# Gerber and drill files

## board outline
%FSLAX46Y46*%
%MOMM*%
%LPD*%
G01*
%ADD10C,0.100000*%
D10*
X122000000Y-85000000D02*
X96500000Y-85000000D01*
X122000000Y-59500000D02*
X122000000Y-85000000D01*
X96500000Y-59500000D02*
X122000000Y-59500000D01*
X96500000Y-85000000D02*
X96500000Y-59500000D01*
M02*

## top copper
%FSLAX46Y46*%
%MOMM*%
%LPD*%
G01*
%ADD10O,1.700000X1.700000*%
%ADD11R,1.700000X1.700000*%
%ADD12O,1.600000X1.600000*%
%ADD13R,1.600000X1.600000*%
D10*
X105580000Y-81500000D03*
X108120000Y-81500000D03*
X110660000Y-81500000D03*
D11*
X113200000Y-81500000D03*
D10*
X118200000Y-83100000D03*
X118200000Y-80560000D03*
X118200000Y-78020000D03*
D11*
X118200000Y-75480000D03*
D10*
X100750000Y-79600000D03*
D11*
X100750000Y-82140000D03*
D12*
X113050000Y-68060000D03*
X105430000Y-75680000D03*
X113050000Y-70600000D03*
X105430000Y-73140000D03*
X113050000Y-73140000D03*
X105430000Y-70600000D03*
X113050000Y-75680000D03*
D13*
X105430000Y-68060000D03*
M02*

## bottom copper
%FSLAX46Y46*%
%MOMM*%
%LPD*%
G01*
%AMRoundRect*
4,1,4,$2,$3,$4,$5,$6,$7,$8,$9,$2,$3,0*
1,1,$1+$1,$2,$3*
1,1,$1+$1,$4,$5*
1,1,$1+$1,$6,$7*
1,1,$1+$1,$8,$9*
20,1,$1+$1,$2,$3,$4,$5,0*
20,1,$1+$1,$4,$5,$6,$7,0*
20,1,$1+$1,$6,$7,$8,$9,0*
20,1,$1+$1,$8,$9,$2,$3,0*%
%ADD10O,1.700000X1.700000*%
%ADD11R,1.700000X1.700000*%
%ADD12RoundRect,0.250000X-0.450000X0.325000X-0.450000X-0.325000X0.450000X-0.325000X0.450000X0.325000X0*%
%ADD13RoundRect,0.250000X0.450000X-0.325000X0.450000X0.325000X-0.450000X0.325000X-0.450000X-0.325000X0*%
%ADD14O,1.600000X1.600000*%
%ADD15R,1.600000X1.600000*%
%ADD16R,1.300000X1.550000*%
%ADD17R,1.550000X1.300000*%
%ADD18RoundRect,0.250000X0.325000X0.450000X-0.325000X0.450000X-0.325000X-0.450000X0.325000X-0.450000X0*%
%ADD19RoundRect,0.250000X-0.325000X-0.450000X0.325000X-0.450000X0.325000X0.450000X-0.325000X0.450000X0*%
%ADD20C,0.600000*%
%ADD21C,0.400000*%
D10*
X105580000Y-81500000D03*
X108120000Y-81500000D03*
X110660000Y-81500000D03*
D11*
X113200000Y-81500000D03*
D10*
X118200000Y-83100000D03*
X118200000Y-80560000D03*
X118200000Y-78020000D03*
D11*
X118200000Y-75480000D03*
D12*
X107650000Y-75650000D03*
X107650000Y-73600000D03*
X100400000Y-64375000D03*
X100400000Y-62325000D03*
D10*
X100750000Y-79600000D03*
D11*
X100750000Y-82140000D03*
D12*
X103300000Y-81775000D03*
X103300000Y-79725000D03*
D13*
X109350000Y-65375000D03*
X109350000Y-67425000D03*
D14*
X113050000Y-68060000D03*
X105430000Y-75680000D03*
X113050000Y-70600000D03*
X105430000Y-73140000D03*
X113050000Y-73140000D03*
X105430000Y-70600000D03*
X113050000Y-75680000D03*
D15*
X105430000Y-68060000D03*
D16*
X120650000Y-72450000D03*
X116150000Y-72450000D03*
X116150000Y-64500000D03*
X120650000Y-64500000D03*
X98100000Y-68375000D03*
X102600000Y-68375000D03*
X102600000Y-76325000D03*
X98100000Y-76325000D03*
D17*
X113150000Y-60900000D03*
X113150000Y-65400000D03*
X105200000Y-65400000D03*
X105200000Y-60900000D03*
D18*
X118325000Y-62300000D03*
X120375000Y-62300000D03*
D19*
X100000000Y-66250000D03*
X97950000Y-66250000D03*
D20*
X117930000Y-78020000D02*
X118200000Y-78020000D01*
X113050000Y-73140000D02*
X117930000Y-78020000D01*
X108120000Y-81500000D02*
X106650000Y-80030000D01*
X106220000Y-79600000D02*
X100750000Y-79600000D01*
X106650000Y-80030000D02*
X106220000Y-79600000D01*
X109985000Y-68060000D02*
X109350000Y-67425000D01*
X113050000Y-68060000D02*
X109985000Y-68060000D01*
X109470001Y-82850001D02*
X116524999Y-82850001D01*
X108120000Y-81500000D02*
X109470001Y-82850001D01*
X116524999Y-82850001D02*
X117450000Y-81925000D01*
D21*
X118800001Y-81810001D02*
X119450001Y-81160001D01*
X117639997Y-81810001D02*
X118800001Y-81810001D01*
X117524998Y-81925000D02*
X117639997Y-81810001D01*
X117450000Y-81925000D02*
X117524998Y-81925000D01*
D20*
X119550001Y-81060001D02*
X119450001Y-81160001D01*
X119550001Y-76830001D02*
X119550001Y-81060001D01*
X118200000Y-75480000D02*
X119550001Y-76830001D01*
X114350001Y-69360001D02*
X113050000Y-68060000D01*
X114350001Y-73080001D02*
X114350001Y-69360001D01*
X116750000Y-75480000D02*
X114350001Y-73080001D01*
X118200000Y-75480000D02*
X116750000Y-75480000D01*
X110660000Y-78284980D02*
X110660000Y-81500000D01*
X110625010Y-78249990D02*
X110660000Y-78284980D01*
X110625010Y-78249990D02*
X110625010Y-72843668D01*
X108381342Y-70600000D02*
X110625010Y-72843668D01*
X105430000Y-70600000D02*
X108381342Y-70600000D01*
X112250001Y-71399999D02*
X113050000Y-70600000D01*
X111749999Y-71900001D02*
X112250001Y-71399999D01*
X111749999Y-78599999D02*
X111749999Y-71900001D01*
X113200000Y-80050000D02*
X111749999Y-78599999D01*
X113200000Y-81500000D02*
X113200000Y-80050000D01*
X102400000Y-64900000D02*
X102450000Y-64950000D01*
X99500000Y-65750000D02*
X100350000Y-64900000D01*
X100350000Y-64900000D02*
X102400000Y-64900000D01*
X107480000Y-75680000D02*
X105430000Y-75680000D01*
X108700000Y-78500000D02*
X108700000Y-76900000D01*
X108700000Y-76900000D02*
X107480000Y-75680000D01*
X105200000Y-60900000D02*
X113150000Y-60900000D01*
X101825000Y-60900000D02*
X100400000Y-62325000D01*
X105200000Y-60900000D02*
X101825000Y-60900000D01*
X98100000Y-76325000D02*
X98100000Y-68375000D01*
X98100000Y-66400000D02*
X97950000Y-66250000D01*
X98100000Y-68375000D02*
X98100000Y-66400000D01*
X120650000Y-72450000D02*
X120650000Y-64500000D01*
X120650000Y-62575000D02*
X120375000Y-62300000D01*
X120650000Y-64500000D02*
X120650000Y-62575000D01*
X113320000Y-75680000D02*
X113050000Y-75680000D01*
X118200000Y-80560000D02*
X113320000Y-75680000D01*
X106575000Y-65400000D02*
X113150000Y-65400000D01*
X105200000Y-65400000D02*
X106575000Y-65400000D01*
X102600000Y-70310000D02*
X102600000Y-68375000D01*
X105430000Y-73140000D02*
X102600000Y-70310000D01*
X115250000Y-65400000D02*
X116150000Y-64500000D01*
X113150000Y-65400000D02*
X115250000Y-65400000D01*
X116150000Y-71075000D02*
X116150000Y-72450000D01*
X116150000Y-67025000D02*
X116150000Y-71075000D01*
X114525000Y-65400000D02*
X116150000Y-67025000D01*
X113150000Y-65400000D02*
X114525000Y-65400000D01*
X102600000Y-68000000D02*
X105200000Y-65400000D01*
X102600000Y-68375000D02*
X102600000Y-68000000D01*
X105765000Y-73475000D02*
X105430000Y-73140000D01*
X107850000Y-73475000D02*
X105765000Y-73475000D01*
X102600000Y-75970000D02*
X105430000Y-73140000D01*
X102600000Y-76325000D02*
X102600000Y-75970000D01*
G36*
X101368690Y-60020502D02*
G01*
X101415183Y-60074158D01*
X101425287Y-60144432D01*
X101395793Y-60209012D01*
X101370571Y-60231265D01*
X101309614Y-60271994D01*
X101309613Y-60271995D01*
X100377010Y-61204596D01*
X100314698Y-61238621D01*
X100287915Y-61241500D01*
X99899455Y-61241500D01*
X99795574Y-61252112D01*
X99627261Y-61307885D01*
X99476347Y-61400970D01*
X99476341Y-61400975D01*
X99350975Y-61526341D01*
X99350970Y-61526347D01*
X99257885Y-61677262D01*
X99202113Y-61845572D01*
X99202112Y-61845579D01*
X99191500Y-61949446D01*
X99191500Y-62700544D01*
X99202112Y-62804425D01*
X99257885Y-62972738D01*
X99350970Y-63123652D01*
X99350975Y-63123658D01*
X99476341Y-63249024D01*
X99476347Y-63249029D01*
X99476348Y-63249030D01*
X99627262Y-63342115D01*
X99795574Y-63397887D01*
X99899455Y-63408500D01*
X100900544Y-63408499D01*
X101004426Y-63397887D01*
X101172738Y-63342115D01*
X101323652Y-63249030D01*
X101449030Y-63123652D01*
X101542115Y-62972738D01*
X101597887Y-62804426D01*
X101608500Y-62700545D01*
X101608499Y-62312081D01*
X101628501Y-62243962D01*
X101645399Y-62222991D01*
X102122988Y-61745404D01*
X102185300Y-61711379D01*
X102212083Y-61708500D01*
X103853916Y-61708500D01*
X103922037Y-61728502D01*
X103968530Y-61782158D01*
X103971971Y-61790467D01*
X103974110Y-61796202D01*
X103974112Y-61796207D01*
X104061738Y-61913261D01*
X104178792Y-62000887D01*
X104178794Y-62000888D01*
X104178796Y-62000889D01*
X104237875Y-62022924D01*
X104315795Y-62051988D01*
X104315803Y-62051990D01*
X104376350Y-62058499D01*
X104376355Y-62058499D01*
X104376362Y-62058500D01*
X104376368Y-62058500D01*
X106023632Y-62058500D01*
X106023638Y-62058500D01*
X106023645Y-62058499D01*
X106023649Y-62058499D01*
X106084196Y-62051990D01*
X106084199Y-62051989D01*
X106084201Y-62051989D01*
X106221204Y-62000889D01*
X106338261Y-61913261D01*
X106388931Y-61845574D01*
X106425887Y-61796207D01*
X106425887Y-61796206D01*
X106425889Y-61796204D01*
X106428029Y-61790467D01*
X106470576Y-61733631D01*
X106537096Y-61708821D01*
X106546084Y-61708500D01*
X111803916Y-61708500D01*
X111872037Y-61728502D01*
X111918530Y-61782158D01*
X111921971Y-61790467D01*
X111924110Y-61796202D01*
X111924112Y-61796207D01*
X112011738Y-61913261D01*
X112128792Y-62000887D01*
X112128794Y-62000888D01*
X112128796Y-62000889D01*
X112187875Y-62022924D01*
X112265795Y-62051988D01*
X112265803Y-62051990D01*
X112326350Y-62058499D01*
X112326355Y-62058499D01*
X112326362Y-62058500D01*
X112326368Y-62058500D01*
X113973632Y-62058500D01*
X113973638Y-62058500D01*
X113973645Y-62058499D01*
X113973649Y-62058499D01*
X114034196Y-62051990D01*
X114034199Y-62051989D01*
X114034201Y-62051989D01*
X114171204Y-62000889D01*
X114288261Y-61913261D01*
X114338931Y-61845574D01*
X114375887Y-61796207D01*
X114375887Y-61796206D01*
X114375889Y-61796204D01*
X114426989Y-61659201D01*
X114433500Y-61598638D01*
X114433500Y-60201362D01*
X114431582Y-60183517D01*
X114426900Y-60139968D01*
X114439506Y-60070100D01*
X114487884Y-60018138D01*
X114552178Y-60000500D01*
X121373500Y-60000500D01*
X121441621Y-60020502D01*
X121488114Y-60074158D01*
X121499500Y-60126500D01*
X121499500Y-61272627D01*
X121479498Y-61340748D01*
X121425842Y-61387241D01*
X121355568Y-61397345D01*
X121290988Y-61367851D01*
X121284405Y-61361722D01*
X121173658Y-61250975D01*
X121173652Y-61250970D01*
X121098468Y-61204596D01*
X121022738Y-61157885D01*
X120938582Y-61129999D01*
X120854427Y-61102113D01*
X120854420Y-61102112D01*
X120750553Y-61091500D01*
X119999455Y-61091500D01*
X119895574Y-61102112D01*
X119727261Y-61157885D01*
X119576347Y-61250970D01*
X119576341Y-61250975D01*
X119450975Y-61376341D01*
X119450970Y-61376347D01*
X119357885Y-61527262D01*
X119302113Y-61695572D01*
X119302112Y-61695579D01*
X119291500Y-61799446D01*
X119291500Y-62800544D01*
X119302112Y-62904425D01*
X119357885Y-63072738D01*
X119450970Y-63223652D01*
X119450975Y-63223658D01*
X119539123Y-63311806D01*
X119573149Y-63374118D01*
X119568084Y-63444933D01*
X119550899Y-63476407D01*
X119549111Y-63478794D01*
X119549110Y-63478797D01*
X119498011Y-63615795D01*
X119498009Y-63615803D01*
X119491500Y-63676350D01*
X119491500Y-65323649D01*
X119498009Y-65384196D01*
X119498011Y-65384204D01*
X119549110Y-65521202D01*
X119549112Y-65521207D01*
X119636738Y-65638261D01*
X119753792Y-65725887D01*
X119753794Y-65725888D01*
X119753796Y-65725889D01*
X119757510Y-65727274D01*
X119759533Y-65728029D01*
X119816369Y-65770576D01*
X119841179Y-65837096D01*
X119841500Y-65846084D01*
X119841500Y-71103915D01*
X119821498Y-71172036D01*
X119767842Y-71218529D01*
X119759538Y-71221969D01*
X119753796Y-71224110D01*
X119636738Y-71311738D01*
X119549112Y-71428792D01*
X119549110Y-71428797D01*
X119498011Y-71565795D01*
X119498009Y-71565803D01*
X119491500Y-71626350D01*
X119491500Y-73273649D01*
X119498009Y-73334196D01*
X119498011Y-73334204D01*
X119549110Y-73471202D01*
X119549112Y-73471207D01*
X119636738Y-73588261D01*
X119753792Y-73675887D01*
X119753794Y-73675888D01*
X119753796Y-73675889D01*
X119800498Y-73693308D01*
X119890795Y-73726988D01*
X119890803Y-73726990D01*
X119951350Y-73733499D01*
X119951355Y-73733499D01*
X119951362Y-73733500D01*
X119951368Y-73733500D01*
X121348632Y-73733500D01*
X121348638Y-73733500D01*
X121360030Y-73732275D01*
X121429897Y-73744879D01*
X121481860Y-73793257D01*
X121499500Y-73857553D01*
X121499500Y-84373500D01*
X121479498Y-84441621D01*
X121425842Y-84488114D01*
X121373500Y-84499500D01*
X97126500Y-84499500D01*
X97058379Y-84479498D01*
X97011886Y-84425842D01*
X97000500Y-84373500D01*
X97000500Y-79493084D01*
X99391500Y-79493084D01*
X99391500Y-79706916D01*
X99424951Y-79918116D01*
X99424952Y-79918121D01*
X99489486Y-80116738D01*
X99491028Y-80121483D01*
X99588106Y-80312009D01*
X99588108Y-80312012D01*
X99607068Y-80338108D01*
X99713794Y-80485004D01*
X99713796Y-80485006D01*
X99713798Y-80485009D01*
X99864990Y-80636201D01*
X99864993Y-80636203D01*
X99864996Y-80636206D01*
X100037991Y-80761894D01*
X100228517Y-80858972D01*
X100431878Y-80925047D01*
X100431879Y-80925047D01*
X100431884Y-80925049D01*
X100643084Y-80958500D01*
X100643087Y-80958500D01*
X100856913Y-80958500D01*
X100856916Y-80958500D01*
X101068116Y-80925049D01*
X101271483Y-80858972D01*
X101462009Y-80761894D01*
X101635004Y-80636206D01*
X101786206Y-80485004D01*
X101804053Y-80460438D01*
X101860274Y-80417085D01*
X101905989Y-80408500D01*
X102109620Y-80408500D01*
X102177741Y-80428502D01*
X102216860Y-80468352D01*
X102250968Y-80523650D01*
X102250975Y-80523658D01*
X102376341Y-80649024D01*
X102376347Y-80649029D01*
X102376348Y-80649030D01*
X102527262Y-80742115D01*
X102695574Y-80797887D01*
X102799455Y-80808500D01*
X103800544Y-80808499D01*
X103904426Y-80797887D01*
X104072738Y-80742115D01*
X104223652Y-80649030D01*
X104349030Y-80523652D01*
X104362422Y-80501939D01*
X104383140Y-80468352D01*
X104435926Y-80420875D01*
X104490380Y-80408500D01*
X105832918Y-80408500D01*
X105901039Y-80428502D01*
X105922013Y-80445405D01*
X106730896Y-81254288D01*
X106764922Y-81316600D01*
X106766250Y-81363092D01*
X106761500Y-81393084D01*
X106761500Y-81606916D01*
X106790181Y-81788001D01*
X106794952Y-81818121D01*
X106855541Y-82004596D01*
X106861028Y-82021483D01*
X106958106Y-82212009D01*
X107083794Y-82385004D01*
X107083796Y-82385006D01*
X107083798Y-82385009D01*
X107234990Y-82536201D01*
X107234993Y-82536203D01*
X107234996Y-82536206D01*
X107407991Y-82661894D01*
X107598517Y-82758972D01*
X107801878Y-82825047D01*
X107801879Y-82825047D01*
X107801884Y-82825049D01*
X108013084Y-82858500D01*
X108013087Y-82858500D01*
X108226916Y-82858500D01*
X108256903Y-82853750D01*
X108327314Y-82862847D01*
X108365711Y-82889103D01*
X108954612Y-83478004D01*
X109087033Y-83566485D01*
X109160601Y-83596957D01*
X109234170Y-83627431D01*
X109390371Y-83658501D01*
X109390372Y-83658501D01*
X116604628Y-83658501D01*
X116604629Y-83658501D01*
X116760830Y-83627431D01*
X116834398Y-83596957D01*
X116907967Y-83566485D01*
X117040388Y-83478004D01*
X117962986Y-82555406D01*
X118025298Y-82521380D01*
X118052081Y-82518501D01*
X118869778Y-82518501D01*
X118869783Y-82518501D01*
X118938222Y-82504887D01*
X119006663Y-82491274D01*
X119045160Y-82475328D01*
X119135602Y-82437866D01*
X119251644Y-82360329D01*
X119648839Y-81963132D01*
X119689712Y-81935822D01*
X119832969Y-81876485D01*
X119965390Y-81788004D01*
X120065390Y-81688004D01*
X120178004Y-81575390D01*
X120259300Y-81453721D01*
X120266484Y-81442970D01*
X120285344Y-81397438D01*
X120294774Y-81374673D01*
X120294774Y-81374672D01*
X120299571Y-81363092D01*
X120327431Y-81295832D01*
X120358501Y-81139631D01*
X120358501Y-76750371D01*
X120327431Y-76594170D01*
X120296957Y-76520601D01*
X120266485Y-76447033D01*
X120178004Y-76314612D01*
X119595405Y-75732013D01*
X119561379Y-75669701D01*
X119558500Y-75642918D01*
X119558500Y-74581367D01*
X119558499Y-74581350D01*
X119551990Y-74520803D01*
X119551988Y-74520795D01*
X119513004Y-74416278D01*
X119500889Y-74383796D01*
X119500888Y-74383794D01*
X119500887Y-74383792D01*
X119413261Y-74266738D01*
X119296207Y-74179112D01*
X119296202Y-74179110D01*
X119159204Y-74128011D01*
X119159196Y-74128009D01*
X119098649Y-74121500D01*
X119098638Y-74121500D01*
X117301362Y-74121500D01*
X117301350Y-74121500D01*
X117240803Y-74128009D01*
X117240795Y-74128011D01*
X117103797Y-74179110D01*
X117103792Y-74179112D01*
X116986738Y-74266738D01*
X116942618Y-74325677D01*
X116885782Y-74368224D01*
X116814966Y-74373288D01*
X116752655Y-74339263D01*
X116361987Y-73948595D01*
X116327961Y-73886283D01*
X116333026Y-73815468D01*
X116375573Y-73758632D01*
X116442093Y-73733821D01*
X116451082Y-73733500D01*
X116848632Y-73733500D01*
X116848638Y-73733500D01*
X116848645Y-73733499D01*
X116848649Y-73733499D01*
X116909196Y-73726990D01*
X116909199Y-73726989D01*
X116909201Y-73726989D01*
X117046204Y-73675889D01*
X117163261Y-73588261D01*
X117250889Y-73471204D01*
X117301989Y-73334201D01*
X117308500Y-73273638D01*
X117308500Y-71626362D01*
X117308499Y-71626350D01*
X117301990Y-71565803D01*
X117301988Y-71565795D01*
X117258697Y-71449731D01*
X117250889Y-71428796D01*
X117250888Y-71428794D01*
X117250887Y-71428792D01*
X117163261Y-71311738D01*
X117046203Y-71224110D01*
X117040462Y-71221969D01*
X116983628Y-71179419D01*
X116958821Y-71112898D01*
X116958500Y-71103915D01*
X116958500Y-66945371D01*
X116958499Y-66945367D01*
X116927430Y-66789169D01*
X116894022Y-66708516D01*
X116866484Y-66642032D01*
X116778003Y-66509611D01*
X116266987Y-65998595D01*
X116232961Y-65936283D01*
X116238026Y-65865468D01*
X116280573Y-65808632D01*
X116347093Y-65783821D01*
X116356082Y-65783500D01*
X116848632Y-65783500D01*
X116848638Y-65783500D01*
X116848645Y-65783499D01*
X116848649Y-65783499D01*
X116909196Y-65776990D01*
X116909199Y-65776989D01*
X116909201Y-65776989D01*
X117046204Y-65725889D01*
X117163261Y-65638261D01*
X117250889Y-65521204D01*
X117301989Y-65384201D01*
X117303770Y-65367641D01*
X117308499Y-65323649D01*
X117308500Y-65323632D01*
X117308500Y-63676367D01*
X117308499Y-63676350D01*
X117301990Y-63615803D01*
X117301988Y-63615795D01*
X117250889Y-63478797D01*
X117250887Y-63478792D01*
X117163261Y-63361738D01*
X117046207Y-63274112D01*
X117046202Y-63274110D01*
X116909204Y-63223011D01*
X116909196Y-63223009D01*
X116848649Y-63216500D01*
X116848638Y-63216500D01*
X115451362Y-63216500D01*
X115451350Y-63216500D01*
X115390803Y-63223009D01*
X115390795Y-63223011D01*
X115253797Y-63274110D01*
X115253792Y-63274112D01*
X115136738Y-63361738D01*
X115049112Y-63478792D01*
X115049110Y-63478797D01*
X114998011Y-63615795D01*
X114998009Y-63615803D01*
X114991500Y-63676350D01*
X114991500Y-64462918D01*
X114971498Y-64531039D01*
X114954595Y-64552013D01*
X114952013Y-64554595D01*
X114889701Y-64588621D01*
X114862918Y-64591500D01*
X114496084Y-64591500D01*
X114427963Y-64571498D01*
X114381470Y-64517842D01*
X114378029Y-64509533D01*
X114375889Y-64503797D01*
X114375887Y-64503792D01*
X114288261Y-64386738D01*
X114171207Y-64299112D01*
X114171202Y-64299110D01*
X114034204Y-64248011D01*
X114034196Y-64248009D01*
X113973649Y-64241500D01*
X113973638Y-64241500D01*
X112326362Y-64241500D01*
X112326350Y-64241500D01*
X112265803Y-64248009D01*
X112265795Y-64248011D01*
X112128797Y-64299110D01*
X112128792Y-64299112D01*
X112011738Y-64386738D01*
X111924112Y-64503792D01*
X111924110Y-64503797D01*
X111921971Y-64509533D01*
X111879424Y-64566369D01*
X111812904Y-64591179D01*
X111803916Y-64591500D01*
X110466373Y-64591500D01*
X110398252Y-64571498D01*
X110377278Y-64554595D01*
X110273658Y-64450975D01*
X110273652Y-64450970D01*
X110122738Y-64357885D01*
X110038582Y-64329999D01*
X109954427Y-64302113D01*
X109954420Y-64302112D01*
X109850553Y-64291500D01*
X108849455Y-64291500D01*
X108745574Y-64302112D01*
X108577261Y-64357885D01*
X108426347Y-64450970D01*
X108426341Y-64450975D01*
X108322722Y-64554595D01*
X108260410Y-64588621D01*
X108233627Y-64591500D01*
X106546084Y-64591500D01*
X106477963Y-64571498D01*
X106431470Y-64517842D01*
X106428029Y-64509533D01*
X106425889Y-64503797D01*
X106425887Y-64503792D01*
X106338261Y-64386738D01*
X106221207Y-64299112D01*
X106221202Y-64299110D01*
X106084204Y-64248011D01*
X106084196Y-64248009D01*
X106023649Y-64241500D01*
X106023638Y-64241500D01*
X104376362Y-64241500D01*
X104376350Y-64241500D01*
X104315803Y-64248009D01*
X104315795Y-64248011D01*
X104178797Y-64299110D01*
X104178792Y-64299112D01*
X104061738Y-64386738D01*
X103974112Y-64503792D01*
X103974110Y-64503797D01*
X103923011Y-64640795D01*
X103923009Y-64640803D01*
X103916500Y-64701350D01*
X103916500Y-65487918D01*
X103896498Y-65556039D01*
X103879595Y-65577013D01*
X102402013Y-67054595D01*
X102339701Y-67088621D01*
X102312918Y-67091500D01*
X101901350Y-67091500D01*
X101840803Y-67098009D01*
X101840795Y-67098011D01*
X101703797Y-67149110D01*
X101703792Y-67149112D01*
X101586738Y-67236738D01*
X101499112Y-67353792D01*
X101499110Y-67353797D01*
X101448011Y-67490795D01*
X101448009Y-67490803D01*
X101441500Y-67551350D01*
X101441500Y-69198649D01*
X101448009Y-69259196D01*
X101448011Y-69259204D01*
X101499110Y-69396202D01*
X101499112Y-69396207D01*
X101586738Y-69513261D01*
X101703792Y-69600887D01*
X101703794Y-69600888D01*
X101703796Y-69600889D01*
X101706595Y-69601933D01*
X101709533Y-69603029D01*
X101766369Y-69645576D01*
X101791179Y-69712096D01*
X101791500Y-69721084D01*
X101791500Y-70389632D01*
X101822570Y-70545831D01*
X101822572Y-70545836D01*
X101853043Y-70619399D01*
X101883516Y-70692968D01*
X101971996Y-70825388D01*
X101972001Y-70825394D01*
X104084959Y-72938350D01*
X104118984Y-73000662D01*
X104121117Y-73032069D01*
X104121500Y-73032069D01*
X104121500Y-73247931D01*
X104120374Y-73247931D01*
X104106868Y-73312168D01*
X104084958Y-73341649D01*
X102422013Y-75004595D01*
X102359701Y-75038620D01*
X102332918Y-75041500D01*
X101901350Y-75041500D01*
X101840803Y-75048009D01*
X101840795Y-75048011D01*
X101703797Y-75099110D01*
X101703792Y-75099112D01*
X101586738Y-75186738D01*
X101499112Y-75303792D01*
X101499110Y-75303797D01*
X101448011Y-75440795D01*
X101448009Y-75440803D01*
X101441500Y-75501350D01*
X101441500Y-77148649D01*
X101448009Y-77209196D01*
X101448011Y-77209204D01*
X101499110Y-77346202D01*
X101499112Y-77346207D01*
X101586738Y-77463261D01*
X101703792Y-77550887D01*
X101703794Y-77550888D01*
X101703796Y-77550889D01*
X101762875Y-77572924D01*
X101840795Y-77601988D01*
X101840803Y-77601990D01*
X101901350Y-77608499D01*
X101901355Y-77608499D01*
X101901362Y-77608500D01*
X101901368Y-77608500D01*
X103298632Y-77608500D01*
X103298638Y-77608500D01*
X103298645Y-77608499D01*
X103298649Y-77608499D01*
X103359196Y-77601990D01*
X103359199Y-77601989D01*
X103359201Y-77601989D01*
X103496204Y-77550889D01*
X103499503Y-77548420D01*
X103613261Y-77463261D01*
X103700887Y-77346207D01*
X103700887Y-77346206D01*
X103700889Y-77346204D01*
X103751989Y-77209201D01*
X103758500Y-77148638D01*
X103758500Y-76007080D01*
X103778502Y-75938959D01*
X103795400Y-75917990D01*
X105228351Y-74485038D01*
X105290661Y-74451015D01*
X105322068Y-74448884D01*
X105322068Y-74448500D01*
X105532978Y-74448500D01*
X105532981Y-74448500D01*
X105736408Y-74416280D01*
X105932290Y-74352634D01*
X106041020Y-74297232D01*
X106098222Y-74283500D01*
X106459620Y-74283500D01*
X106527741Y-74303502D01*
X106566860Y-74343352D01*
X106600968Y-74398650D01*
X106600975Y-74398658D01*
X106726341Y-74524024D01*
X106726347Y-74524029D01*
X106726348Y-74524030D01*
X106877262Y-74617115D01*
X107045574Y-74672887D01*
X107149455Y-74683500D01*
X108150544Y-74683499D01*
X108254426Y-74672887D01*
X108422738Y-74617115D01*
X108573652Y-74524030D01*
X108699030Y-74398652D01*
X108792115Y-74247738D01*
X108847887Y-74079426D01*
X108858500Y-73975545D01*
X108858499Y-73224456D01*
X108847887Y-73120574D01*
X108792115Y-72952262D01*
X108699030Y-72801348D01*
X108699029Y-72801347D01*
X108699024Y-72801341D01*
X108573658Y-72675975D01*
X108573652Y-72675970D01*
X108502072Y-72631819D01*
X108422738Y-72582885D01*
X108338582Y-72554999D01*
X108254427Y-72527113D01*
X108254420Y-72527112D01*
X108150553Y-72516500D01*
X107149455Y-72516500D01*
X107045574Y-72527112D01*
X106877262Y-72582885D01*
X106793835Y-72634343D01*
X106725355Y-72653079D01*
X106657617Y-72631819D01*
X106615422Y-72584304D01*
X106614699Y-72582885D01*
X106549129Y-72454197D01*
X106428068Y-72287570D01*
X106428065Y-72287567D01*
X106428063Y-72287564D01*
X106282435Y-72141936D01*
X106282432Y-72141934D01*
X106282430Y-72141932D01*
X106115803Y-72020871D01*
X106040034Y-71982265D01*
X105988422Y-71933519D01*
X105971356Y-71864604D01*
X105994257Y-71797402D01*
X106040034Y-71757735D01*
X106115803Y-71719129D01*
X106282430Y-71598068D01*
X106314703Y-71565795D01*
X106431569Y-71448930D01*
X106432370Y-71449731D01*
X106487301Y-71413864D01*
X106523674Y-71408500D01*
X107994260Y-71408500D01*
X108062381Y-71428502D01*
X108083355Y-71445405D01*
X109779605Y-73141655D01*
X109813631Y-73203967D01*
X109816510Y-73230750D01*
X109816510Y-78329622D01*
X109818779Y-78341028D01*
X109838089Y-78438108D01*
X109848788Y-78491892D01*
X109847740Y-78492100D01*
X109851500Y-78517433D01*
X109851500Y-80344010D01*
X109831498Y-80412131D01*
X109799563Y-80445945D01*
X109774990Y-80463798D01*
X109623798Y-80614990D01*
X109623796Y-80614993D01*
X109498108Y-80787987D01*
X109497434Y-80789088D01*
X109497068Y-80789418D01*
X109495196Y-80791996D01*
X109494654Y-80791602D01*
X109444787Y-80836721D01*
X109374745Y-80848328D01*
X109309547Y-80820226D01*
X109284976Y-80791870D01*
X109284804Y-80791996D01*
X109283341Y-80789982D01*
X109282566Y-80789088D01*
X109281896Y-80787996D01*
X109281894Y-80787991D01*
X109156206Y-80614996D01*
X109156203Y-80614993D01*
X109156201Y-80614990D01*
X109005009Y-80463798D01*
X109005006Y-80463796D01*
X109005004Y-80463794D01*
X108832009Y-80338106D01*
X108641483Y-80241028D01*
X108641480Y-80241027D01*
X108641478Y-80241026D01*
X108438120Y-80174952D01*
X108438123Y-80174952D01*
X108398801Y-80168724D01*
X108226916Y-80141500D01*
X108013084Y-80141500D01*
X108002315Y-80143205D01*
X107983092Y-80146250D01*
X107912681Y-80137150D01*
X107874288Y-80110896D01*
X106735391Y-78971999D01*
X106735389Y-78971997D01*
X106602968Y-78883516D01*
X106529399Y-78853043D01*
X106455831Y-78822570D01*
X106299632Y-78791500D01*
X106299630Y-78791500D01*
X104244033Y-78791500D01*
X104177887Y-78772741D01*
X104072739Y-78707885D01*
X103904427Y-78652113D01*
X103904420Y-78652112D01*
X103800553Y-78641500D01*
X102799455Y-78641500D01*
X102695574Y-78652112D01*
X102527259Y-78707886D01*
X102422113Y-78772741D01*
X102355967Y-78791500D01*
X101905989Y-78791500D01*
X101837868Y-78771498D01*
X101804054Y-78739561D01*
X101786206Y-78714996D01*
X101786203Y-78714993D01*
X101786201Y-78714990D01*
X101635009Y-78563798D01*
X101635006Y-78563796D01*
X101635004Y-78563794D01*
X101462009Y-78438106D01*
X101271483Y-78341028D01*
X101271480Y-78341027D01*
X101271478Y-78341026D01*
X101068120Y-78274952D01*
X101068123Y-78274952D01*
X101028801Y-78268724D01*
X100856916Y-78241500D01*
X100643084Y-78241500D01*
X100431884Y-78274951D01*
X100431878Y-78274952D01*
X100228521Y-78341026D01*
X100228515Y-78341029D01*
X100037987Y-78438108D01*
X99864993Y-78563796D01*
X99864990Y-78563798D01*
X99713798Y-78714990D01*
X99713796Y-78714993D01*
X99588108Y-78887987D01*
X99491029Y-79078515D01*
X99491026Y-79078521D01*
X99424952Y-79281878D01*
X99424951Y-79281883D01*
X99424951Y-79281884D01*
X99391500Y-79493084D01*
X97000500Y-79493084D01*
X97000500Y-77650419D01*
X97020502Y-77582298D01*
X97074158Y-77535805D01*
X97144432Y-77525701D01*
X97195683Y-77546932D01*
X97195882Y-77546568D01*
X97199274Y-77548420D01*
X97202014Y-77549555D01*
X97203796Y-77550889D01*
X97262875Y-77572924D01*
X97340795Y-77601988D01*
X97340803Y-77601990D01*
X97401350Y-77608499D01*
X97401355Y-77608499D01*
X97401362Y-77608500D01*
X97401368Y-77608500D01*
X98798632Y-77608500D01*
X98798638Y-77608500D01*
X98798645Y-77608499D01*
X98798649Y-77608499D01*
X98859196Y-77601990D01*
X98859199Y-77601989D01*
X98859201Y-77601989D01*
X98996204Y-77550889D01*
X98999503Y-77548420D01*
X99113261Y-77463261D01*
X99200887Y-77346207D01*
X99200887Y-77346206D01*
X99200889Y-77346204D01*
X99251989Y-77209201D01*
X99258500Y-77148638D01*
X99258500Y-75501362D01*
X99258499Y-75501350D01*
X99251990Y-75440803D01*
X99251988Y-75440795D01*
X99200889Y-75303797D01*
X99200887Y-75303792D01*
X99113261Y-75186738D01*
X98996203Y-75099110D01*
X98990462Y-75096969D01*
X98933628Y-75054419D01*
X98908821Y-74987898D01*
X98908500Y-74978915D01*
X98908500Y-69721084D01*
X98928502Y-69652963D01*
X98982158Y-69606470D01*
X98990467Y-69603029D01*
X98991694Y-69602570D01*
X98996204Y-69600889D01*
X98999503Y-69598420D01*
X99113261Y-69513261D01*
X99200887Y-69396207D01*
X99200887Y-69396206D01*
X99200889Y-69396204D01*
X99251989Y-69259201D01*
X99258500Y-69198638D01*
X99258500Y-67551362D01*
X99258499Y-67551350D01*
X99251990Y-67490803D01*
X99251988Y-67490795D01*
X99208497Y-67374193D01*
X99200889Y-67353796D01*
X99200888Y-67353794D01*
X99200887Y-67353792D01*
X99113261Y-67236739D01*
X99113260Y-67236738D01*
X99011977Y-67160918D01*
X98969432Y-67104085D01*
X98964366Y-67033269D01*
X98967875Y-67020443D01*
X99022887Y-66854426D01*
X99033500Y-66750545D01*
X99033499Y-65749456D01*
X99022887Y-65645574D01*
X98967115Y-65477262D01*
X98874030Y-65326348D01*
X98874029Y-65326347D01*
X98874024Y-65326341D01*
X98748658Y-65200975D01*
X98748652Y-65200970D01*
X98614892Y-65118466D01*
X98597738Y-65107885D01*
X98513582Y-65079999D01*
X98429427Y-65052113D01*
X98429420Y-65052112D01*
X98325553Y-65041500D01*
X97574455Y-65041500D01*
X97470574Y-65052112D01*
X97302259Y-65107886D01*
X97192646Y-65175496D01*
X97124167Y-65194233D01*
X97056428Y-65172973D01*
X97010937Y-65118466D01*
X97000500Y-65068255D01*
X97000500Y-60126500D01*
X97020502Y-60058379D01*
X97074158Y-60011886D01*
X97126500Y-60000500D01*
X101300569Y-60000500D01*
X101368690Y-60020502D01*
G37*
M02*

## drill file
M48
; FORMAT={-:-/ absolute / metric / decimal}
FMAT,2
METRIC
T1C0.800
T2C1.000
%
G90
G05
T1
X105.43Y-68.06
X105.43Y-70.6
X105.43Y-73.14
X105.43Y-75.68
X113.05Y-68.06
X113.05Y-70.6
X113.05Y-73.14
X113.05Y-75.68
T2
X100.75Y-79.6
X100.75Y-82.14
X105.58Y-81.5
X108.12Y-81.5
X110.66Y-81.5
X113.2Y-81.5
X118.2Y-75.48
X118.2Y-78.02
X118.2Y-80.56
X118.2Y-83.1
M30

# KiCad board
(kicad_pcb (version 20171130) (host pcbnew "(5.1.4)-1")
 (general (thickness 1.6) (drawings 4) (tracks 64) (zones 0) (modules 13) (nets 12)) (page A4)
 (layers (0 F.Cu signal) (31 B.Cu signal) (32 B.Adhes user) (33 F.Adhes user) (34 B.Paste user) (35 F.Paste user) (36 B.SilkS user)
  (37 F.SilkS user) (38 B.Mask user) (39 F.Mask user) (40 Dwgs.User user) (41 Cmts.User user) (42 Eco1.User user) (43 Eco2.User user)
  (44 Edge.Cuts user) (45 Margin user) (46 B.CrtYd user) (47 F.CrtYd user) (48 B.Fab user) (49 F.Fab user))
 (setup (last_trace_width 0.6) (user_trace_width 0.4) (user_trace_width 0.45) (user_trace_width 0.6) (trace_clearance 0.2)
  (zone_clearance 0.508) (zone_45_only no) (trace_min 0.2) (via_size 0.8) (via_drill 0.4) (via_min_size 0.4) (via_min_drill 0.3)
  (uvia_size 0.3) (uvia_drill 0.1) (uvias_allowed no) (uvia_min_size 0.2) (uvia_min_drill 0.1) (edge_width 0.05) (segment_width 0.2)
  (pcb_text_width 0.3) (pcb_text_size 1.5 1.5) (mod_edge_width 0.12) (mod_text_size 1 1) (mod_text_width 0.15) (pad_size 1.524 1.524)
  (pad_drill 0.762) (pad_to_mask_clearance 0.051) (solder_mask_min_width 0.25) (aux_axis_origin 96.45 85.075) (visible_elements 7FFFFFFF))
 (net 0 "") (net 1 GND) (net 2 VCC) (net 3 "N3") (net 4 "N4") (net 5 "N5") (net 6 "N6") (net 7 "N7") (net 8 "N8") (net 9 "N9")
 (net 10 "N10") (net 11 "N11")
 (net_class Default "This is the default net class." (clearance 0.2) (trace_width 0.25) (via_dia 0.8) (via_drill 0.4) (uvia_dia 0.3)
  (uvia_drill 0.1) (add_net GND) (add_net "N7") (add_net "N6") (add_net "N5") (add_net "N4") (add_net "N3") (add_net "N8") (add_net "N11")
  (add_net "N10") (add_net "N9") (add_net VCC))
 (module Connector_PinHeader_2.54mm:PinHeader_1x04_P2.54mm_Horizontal (layer F.Cu) (at 113.2 81.5 270)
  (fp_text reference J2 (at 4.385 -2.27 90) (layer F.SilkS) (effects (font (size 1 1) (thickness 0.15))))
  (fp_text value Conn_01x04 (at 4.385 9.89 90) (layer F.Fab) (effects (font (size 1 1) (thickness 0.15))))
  (pad 4 thru_hole oval (at 0 7.62 270) (size 1.7 1.7) (drill 1) (layers *.Cu *.Mask) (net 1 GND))
  (pad 3 thru_hole oval (at 0 5.08 270) (size 1.7 1.7) (drill 1) (layers *.Cu *.Mask) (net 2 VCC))
  (pad 2 thru_hole oval (at 0 2.54 270) (size 1.7 1.7) (drill 1) (layers *.Cu *.Mask) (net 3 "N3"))
  (pad 1 thru_hole rect (at 0 0 270) (size 1.7 1.7) (drill 1) (layers *.Cu *.Mask) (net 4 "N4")))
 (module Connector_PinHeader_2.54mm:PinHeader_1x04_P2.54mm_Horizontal (layer F.Cu) (at 118.2 75.48)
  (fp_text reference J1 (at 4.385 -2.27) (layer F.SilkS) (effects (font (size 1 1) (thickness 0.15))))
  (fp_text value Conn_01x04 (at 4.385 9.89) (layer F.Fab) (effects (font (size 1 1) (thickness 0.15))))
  (pad 4 thru_hole oval (at 0 7.62) (size 1.7 1.7) (drill 1) (layers *.Cu *.Mask) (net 1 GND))
  (pad 3 thru_hole oval (at 0 5.08) (size 1.7 1.7) (drill 1) (layers *.Cu *.Mask) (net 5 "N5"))
  (pad 2 thru_hole oval (at 0 2.54) (size 1.7 1.7) (drill 1) (layers *.Cu *.Mask) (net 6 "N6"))
  (pad 1 thru_hole rect (at 0 0) (size 1.7 1.7) (drill 1) (layers *.Cu *.Mask) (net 2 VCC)))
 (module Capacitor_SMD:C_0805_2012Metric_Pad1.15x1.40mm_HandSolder (layer B.Cu) (at 107.65 74.625 270)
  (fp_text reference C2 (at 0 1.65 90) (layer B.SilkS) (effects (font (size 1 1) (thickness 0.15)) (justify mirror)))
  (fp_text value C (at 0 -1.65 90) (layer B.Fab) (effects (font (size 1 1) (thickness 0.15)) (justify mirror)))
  (pad 2 smd roundrect (at 1.025 0 270) (size 1.15 1.4) (layers B.Cu B.Paste B.Mask) (roundrect_rratio 0.217391) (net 1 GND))
  (pad 1 smd roundrect (at -1.025 0 270) (size 1.15 1.4) (layers B.Cu B.Paste B.Mask) (roundrect_rratio 0.217391) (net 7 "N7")))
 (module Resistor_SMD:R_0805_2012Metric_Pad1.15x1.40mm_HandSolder (layer B.Cu) (at 100.4 63.35 270)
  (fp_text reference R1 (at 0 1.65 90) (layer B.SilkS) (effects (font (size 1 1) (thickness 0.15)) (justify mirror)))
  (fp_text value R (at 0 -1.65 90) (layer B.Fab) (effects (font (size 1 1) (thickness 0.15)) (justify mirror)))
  (pad 2 smd roundrect (at 1.025 0 270) (size 1.15 1.4) (layers B.Cu B.Paste B.Mask) (roundrect_rratio 0.217391) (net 1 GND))
  (pad 1 smd roundrect (at -1.025 0 270) (size 1.15 1.4) (layers B.Cu B.Paste B.Mask) (roundrect_rratio 0.217391) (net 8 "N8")))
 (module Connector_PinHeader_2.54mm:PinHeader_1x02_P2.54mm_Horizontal (layer F.Cu) (at 100.75 82.14 180)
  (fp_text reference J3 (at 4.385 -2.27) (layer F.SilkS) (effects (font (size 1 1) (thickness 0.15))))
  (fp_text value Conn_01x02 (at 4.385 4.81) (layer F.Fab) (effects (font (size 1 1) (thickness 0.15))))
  (pad 2 thru_hole oval (at 0 2.54 180) (size 1.7 1.7) (drill 1) (layers *.Cu *.Mask) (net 2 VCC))
  (pad 1 thru_hole rect (at 0 0 180) (size 1.7 1.7) (drill 1) (layers *.Cu *.Mask) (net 1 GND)))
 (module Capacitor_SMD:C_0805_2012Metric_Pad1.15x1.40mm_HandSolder (layer B.Cu) (at 103.3 80.75 270)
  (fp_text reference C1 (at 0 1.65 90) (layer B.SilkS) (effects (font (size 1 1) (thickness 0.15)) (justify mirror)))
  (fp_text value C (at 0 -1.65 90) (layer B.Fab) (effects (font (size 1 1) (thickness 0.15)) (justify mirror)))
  (pad 2 smd roundrect (at 1.025 0 270) (size 1.15 1.4) (layers B.Cu B.Paste B.Mask) (roundrect_rratio 0.217391) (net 1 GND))
  (pad 1 smd roundrect (at -1.025 0 270) (size 1.15 1.4) (layers B.Cu B.Paste B.Mask) (roundrect_rratio 0.217391) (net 2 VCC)))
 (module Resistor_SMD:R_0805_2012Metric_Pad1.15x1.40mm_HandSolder (layer B.Cu) (at 109.35 66.4 90)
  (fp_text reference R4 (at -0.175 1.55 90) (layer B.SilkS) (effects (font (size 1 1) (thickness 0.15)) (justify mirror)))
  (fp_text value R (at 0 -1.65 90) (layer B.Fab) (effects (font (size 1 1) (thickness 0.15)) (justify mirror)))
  (pad 2 smd roundrect (at 1.025 0 90) (size 1.15 1.4) (layers B.Cu B.Paste B.Mask) (roundrect_rratio 0.217391) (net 7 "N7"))
  (pad 1 smd roundrect (at -1.025 0 90) (size 1.15 1.4) (layers B.Cu B.Paste B.Mask) (roundrect_rratio 0.217391) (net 2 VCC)))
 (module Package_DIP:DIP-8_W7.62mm (layer F.Cu) (at 105.43 68.06)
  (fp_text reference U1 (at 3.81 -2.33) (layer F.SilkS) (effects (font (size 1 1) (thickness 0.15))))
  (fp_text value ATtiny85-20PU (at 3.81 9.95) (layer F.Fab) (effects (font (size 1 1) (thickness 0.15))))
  (pad 8 thru_hole oval (at 7.62 0) (size 1.6 1.6) (drill 0.8) (layers *.Cu *.Mask) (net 2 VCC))
  (pad 4 thru_hole oval (at 0 7.62) (size 1.6 1.6) (drill 0.8) (layers *.Cu *.Mask) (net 1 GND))
  (pad 7 thru_hole oval (at 7.62 2.54) (size 1.6 1.6) (drill 0.8) (layers *.Cu *.Mask) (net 4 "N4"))
  (pad 3 thru_hole oval (at 0 5.08) (size 1.6 1.6) (drill 0.8) (layers *.Cu *.Mask) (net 7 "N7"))
  (pad 6 thru_hole oval (at 7.62 5.08) (size 1.6 1.6) (drill 0.8) (layers *.Cu *.Mask) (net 6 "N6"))
  (pad 2 thru_hole oval (at 0 2.54) (size 1.6 1.6) (drill 0.8) (layers *.Cu *.Mask) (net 3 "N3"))
  (pad 5 thru_hole oval (at 7.62 7.62) (size 1.6 1.6) (drill 0.8) (layers *.Cu *.Mask) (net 5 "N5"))
  (pad 1 thru_hole rect (at 0 0) (size 1.6 1.6) (drill 0.8) (layers *.Cu *.Mask) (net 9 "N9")))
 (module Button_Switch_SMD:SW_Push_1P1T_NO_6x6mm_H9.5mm (layer B.Cu) (at 118.4 68.475 270)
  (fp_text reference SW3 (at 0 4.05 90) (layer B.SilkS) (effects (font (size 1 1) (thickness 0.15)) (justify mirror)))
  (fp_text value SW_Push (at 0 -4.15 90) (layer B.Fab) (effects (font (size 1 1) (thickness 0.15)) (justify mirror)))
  (pad 2 smd rect (at 3.975 -2.25 270) (size 1.55 1.3) (layers B.Cu B.Paste B.Mask) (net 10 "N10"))
  (pad 1 smd rect (at 3.975 2.25 270) (size 1.55 1.3) (layers B.Cu B.Paste B.Mask) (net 7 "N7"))
  (pad 1 smd rect (at -3.975 2.25 270) (size 1.55 1.3) (layers B.Cu B.Paste B.Mask) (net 7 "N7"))
  (pad 2 smd rect (at -3.975 -2.25 270) (size 1.55 1.3) (layers B.Cu B.Paste B.Mask) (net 10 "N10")))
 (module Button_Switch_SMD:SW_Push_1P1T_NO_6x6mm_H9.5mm (layer B.Cu) (at 100.35 72.35 90)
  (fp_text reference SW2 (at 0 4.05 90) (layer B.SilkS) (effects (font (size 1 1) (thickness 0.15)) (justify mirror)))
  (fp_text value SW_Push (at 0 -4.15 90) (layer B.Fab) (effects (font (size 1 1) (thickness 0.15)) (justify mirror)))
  (pad 2 smd rect (at 3.975 -2.25 90) (size 1.55 1.3) (layers B.Cu B.Paste B.Mask) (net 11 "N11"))
  (pad 1 smd rect (at 3.975 2.25 90) (size 1.55 1.3) (layers B.Cu B.Paste B.Mask) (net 7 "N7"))
  (pad 1 smd rect (at -3.975 2.25 90) (size 1.55 1.3) (layers B.Cu B.Paste B.Mask) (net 7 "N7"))
  (pad 2 smd rect (at -3.975 -2.25 90) (size 1.55 1.3) (layers B.Cu B.Paste B.Mask) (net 11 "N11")))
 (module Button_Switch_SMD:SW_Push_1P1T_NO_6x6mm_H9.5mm (layer B.Cu) (at 109.175 63.15)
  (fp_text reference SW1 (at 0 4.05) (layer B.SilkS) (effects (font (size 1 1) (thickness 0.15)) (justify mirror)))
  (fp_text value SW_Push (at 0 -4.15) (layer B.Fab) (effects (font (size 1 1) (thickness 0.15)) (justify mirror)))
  (pad 2 smd rect (at 3.975 -2.25) (size 1.55 1.3) (layers B.Cu B.Paste B.Mask) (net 8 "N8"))
  (pad 1 smd rect (at 3.975 2.25) (size 1.55 1.3) (layers B.Cu B.Paste B.Mask) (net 7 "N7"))
  (pad 1 smd rect (at -3.975 2.25) (size 1.55 1.3) (layers B.Cu B.Paste B.Mask) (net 7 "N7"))
  (pad 2 smd rect (at -3.975 -2.25) (size 1.55 1.3) (layers B.Cu B.Paste B.Mask) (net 8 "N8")))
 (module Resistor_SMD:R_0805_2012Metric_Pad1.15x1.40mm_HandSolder (layer B.Cu) (at 119.35 62.3 180)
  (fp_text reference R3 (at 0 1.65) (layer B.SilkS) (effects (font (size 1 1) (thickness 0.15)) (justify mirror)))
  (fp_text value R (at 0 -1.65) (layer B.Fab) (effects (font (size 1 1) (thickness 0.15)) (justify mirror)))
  (pad 2 smd roundrect (at 1.025 0 180) (size 1.15 1.4) (layers B.Cu B.Paste B.Mask) (roundrect_rratio 0.217391) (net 1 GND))
  (pad 1 smd roundrect (at -1.025 0 180) (size 1.15 1.4) (layers B.Cu B.Paste B.Mask) (roundrect_rratio 0.217391) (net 10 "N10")))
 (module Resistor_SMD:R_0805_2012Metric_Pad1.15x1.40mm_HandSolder (layer B.Cu) (at 98.975 66.25)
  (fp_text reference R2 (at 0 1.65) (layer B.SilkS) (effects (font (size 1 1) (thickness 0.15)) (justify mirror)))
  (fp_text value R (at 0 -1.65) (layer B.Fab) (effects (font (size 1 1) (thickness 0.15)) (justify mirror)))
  (pad 2 smd roundrect (at 1.025 0) (size 1.15 1.4) (layers B.Cu B.Paste B.Mask) (roundrect_rratio 0.217391) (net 1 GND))
  (pad 1 smd roundrect (at -1.025 0) (size 1.15 1.4) (layers B.Cu B.Paste B.Mask) (roundrect_rratio 0.217391) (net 11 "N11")))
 (gr_line (start 122 85) (end 96.5 85) (layer Edge.Cuts) (width 0.1))
 (gr_line (start 122 59.5) (end 122 85) (layer Edge.Cuts) (width 0.1))
 (gr_line (start 96.5 59.5) (end 122 59.5) (layer Edge.Cuts) (width 0.1))
 (gr_line (start 96.5 85) (end 96.5 59.5) (layer Edge.Cuts) (width 0.1))
 (segment (start 117.93 78.02) (end 118.2 78.02) (width 0.6) (layer B.Cu) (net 6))
 (segment (start 113.05 73.14) (end 117.93 78.02) (width 0.6) (layer B.Cu) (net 6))
 (segment (start 108.12 81.5) (end 106.65 80.03) (width 0.6) (layer B.Cu) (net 2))
 (segment (start 106.22 79.6) (end 100.75 79.6) (width 0.6) (layer B.Cu) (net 2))
 (segment (start 106.65 80.03) (end 106.22 79.6) (width 0.6) (layer B.Cu) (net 2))
 (segment (start 109.985 68.06) (end 109.35 67.425) (width 0.6) (layer B.Cu) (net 2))
 (segment (start 113.05 68.06) (end 109.985 68.06) (width 0.6) (layer B.Cu) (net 2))
 (segment (start 109.470001 82.850001) (end 116.524999 82.850001) (width 0.6) (layer B.Cu) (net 2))
 (segment (start 108.12 81.5) (end 109.470001 82.850001) (width 0.6) (layer B.Cu) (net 2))
 (segment (start 116.524999 82.850001) (end 117.45 81.925) (width 0.6) (layer B.Cu) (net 2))
 (segment (start 118.800001 81.810001) (end 119.450001 81.160001) (width 0.4) (layer B.Cu) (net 2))
 (segment (start 117.639997 81.810001) (end 118.800001 81.810001) (width 0.4) (layer B.Cu) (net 2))
 (segment (start 117.524998 81.925) (end 117.639997 81.810001) (width 0.4) (layer B.Cu) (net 2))
 (segment (start 117.45 81.925) (end 117.524998 81.925) (width 0.4) (layer B.Cu) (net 2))
 (segment (start 119.550001 81.060001) (end 119.450001 81.160001) (width 0.6) (layer B.Cu) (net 2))
 (segment (start 119.550001 76.830001) (end 119.550001 81.060001) (width 0.6) (layer B.Cu) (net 2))
 (segment (start 118.2 75.48) (end 119.550001 76.830001) (width 0.6) (layer B.Cu) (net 2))
 (segment (start 114.350001 69.360001) (end 113.05 68.06) (width 0.6) (layer B.Cu) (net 2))
 (segment (start 114.350001 73.080001) (end 114.350001 69.360001) (width 0.6) (layer B.Cu) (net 2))
 (segment (start 116.75 75.48) (end 114.350001 73.080001) (width 0.6) (layer B.Cu) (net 2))
 (segment (start 118.2 75.48) (end 116.75 75.48) (width 0.6) (layer B.Cu) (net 2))
 (segment (start 110.66 78.28498) (end 110.66 81.5) (width 0.6) (layer B.Cu) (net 3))
 (segment (start 110.62501 78.24999) (end 110.66 78.28498) (width 0.6) (layer B.Cu) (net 3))
 (segment (start 110.62501 78.24999) (end 110.62501 72.843668) (width 0.6) (layer B.Cu) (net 3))
 (segment (start 108.381342 70.6) (end 110.62501 72.843668) (width 0.6) (layer B.Cu) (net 3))
 (segment (start 105.43 70.6) (end 108.381342 70.6) (width 0.6) (layer B.Cu) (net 3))
 (segment (start 112.250001 71.399999) (end 113.05 70.6) (width 0.6) (layer B.Cu) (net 4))
 (segment (start 111.749999 71.900001) (end 112.250001 71.399999) (width 0.6) (layer B.Cu) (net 4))
 (segment (start 111.749999 78.599999) (end 111.749999 71.900001) (width 0.6) (layer B.Cu) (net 4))
 (segment (start 113.2 80.05) (end 111.749999 78.599999) (width 0.6) (layer B.Cu) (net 4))
 (segment (start 113.2 81.5) (end 113.2 80.05) (width 0.6) (layer B.Cu) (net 4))
 (segment (start 102.4 64.9) (end 102.45 64.95) (width 0.6) (layer B.Cu) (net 1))
 (segment (start 99.5 65.75) (end 100.35 64.9) (width 0.6) (layer B.Cu) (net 1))
 (segment (start 100.35 64.9) (end 102.4 64.9) (width 0.6) (layer B.Cu) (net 1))
 (segment (start 107.48 75.68) (end 105.43 75.68) (width 0.6) (layer B.Cu) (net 1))
 (segment (start 108.7 78.5) (end 108.7 76.9) (width 0.6) (layer B.Cu) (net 1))
 (segment (start 108.7 76.9) (end 107.48 75.68) (width 0.6) (layer B.Cu) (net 1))
 (segment (start 105.2 60.9) (end 113.15 60.9) (width 0.6) (layer B.Cu) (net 8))
 (segment (start 101.825 60.9) (end 100.4 62.325) (width 0.6) (layer B.Cu) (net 8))
 (segment (start 105.2 60.9) (end 101.825 60.9) (width 0.6) (layer B.Cu) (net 8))
 (segment (start 98.1 76.325) (end 98.1 68.375) (width 0.6) (layer B.Cu) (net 11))
 (segment (start 98.1 66.4) (end 97.95 66.25) (width 0.6) (layer B.Cu) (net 11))
 (segment (start 98.1 68.375) (end 98.1 66.4) (width 0.6) (layer B.Cu) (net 11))
 (segment (start 120.65 72.45) (end 120.65 64.5) (width 0.6) (layer B.Cu) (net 10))
 (segment (start 120.65 62.575) (end 120.375 62.3) (width 0.6) (layer B.Cu) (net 10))
 (segment (start 120.65 64.5) (end 120.65 62.575) (width 0.6) (layer B.Cu) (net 10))
 (segment (start 113.32 75.68) (end 113.05 75.68) (width 0.6) (layer B.Cu) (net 5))
 (segment (start 118.2 80.56) (end 113.32 75.68) (width 0.6) (layer B.Cu) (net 5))
 (segment (start 106.575 65.4) (end 113.15 65.4) (width 0.6) (layer B.Cu) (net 7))
 (segment (start 105.2 65.4) (end 106.575 65.4) (width 0.6) (layer B.Cu) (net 7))
 (segment (start 102.6 70.31) (end 102.6 68.375) (width 0.6) (layer B.Cu) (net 7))
 (segment (start 105.43 73.14) (end 102.6 70.31) (width 0.6) (layer B.Cu) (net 7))
 (segment (start 115.25 65.4) (end 116.15 64.5) (width 0.6) (layer B.Cu) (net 7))
 (segment (start 113.15 65.4) (end 115.25 65.4) (width 0.6) (layer B.Cu) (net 7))
 (segment (start 116.15 71.075) (end 116.15 72.45) (width 0.6) (layer B.Cu) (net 7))
 (segment (start 116.15 67.025) (end 116.15 71.075) (width 0.6) (layer B.Cu) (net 7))
 (segment (start 114.525 65.4) (end 116.15 67.025) (width 0.6) (layer B.Cu) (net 7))
 (segment (start 113.15 65.4) (end 114.525 65.4) (width 0.6) (layer B.Cu) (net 7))
 (segment (start 102.6 68) (end 105.2 65.4) (width 0.6) (layer B.Cu) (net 7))
 (segment (start 102.6 68.375) (end 102.6 68) (width 0.6) (layer B.Cu) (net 7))
 (segment (start 105.765 73.475) (end 105.43 73.14) (width 0.6) (layer B.Cu) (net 7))
 (segment (start 107.85 73.475) (end 105.765 73.475) (width 0.6) (layer B.Cu) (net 7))
 (segment (start 102.6 75.97) (end 105.43 73.14) (width 0.6) (layer B.Cu) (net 7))
 (segment (start 102.6 76.325) (end 102.6 75.97) (width 0.6) (layer B.Cu) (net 7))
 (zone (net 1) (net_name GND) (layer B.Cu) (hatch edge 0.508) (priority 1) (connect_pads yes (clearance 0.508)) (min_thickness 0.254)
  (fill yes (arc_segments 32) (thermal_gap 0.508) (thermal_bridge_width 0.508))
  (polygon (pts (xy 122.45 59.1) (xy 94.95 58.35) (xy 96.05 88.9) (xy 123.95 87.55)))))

